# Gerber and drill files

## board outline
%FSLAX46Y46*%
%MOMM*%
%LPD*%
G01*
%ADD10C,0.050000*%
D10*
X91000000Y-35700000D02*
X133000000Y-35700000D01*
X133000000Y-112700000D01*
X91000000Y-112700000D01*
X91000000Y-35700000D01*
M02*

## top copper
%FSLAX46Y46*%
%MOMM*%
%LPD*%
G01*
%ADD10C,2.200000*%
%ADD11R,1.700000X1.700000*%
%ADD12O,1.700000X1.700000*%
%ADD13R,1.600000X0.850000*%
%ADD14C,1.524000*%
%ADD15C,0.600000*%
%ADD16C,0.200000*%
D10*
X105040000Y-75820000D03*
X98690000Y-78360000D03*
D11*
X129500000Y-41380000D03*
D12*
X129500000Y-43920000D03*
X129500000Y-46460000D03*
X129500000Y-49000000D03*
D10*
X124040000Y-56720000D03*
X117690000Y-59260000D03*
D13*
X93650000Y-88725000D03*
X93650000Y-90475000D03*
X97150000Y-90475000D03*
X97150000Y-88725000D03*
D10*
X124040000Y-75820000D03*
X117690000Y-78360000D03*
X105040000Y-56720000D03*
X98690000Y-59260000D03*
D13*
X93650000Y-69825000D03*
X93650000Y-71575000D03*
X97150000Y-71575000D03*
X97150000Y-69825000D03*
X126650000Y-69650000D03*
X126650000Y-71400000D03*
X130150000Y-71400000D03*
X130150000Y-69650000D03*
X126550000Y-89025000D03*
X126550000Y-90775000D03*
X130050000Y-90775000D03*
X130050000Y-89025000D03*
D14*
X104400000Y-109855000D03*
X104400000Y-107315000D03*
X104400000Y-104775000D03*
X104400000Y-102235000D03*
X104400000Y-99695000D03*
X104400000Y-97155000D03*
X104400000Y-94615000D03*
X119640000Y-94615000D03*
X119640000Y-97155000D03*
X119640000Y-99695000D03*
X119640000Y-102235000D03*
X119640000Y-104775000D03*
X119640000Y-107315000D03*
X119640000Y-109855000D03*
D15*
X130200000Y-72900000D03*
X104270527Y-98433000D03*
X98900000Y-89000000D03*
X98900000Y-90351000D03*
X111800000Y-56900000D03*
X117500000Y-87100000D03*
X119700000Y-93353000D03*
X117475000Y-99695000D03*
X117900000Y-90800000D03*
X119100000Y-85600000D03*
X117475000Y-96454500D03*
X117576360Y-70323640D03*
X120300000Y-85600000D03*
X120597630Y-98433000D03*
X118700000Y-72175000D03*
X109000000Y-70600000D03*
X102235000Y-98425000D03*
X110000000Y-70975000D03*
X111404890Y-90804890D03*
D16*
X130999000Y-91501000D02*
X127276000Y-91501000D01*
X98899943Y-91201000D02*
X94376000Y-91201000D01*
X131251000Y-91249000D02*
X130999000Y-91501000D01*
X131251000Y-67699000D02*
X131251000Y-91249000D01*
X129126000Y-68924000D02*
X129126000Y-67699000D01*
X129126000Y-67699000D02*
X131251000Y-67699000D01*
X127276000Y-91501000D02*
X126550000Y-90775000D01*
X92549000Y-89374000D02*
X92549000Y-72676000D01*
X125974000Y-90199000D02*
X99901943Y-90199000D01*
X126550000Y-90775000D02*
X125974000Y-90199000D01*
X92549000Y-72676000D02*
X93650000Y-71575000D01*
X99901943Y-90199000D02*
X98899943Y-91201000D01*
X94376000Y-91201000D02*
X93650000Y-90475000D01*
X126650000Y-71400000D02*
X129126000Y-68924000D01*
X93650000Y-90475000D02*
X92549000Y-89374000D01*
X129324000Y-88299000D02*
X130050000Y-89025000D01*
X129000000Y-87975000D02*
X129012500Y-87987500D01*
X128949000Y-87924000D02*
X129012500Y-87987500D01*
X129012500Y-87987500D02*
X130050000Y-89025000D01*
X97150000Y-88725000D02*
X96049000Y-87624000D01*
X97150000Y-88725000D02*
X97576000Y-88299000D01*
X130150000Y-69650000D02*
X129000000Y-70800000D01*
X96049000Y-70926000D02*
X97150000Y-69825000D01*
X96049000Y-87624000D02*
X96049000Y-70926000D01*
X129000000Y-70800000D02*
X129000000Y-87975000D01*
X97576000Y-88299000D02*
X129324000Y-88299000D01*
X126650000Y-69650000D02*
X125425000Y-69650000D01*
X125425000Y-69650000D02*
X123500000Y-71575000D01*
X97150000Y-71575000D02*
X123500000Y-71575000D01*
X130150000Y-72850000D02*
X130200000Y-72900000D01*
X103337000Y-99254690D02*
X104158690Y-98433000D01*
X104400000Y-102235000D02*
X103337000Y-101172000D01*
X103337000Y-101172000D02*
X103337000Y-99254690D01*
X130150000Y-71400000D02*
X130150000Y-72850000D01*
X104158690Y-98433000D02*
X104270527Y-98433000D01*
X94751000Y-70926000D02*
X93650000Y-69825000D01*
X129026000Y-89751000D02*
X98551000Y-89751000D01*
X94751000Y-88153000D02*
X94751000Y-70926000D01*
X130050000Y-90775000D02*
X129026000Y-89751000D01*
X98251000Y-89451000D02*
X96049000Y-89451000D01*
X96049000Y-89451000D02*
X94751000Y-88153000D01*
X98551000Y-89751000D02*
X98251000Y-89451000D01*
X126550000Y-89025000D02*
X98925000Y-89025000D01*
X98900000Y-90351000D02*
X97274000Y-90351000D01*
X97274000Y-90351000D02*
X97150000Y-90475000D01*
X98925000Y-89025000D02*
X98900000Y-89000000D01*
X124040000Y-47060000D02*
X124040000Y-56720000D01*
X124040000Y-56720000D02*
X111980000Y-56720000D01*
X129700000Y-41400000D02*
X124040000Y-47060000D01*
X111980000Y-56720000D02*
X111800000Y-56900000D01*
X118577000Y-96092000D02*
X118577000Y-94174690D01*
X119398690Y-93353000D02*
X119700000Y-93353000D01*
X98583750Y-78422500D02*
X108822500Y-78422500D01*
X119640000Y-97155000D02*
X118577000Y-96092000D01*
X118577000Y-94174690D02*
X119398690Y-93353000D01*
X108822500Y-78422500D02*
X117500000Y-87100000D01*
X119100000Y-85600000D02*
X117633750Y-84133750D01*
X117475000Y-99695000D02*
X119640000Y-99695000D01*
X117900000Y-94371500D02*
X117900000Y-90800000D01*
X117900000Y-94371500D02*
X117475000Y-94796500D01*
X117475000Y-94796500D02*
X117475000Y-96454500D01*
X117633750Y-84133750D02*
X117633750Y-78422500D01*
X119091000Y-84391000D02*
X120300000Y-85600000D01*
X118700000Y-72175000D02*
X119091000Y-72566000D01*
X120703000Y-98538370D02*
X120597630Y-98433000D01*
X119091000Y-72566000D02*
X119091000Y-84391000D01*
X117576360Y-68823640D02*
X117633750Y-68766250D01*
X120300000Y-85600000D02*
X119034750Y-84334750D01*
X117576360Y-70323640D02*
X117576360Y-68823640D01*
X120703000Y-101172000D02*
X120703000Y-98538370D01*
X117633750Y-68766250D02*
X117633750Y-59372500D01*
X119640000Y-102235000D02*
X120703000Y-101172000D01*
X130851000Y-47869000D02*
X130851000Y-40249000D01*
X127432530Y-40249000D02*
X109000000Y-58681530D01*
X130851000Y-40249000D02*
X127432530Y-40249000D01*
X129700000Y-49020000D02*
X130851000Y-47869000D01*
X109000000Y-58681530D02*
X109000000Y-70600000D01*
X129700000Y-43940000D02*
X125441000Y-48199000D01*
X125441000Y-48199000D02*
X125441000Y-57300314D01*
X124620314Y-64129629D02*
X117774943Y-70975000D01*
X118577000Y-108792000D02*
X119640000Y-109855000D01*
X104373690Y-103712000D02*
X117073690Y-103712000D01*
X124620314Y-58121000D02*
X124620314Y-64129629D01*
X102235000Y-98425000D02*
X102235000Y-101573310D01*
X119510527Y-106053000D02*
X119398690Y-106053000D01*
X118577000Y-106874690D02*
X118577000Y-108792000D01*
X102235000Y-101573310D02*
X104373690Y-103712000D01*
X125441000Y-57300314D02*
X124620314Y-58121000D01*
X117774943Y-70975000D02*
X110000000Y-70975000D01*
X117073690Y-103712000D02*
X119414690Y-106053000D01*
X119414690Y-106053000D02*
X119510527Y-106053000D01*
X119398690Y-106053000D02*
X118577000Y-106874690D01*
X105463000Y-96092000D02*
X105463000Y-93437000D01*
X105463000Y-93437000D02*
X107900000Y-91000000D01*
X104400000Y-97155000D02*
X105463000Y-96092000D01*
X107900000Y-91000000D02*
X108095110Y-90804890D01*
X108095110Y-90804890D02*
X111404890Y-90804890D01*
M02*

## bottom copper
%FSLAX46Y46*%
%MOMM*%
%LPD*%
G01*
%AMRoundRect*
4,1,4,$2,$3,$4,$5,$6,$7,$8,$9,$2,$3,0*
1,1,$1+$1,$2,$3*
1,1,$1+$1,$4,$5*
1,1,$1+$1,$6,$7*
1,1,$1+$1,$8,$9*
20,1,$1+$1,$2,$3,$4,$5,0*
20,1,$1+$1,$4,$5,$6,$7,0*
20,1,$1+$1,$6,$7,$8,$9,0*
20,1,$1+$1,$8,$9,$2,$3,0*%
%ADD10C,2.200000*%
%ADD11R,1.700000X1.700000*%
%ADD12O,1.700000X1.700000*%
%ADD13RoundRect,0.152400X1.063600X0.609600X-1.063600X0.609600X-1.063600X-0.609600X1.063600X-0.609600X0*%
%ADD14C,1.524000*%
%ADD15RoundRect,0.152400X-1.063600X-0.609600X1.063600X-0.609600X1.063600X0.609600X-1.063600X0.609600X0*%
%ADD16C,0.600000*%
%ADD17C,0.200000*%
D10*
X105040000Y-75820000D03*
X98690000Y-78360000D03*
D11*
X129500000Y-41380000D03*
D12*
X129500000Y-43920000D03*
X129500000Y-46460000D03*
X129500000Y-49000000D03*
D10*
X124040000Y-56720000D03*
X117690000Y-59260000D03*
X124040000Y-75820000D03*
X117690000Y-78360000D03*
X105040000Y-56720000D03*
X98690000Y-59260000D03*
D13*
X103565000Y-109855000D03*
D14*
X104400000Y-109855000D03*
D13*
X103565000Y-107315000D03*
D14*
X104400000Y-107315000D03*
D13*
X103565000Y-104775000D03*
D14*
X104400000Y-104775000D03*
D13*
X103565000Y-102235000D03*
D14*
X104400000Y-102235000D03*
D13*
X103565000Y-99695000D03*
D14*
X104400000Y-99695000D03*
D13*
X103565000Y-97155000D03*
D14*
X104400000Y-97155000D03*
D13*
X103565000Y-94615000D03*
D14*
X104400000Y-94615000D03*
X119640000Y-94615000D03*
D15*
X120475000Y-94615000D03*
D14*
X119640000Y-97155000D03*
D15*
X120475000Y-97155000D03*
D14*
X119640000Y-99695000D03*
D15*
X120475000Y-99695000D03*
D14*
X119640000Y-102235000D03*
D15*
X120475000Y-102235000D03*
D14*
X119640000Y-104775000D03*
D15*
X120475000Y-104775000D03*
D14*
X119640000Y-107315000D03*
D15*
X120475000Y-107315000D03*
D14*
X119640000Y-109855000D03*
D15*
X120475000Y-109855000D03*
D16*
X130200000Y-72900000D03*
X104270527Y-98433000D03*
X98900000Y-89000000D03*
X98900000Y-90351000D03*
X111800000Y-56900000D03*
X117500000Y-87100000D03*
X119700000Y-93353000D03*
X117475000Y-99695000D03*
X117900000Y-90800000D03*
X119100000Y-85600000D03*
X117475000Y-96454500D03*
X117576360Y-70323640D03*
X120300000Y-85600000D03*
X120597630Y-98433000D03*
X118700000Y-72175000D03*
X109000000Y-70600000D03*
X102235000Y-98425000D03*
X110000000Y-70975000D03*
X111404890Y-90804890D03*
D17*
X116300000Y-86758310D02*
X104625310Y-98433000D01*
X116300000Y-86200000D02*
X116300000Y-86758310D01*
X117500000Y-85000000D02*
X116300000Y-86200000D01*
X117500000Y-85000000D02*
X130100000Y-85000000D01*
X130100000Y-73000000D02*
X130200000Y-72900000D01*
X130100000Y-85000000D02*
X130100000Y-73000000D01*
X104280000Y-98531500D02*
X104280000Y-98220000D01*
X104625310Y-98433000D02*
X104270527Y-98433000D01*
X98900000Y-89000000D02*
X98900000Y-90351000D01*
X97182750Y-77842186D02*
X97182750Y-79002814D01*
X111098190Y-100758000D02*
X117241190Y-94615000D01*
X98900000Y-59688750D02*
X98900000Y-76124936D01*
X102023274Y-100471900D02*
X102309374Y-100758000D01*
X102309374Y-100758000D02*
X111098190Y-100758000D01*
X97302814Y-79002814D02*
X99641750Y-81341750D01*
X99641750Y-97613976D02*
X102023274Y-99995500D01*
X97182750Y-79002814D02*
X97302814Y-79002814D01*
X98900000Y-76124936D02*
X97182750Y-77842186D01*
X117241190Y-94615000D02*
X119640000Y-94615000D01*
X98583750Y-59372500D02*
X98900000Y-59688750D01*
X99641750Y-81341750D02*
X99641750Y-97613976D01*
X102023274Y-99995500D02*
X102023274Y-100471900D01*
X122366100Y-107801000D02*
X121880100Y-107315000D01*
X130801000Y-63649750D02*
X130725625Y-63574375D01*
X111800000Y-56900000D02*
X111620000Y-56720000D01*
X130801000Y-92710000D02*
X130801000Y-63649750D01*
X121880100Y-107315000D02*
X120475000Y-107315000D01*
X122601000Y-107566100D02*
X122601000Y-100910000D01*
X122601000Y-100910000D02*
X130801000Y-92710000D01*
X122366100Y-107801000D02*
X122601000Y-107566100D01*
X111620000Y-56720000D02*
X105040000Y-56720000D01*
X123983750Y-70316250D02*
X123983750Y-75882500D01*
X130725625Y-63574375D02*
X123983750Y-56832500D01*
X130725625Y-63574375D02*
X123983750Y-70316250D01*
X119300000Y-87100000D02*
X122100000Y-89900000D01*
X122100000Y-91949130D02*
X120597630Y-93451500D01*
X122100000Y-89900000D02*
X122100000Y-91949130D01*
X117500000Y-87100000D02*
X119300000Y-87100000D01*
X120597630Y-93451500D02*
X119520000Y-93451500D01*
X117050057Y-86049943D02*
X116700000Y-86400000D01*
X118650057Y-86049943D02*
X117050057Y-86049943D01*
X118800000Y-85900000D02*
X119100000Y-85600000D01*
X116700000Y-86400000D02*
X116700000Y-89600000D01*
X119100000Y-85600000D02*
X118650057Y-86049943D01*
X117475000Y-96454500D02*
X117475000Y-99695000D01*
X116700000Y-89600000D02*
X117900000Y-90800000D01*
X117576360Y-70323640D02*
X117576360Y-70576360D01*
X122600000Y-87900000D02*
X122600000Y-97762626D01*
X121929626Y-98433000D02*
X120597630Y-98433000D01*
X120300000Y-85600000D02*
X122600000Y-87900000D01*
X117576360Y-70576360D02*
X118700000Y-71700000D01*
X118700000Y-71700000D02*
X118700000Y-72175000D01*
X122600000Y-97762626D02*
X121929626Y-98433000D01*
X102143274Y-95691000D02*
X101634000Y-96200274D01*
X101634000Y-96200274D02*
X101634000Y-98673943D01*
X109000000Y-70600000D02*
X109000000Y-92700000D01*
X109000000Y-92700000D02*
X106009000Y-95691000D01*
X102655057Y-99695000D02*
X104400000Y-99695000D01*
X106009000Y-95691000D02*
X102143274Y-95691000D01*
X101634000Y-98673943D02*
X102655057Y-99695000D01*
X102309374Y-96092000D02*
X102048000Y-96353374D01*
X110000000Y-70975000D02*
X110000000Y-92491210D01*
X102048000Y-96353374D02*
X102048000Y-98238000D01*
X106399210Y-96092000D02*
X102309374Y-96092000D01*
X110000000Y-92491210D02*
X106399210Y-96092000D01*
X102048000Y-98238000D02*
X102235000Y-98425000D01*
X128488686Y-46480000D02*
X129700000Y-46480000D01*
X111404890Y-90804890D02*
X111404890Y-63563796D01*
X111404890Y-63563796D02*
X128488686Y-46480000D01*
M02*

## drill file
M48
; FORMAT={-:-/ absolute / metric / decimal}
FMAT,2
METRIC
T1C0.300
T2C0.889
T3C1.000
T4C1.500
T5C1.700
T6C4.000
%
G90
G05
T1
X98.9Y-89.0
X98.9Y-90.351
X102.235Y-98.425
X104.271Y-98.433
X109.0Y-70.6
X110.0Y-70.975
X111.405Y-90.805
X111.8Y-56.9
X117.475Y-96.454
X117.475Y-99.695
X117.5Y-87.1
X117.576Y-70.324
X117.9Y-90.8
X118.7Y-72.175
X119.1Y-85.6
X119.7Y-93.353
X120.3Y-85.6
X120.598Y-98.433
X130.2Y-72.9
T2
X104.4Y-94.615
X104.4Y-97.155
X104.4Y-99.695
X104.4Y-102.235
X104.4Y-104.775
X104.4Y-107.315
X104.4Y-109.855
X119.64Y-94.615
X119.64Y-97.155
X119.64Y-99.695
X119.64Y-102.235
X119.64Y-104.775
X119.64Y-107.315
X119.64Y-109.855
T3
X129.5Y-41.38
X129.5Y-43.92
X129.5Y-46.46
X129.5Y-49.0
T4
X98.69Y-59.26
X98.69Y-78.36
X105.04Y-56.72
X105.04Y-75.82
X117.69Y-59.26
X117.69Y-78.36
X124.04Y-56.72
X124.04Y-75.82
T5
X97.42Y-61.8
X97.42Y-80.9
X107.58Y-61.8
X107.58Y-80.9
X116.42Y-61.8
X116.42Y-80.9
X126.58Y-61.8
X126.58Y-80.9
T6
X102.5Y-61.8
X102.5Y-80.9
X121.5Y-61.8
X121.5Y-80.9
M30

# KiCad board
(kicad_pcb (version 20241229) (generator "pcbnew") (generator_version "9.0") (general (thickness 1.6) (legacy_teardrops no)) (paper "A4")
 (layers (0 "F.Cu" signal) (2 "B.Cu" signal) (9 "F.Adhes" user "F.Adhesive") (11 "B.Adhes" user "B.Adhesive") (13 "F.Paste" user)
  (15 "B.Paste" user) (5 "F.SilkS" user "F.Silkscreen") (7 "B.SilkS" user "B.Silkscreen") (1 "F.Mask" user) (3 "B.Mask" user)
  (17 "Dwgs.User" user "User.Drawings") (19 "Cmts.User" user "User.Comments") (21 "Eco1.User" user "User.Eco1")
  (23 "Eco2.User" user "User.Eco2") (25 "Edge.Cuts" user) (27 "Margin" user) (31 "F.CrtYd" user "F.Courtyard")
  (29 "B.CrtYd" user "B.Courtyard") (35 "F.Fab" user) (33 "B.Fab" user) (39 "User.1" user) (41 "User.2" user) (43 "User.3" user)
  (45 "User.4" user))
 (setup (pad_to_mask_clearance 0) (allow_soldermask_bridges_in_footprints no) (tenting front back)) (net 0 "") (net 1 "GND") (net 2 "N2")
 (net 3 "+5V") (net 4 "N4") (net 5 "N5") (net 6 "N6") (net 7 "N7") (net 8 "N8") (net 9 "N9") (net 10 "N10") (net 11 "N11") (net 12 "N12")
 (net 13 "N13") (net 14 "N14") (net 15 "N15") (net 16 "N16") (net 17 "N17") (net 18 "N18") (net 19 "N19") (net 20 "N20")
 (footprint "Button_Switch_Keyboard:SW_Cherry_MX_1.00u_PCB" (layer "F.Cu") (at 105.04 75.82)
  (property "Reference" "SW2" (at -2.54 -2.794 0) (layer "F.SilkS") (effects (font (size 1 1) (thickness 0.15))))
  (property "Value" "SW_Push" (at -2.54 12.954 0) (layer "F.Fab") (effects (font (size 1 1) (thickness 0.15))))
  (pad "" np_thru_hole circle (at -7.62 5.08) (size 1.7 1.7) (drill 1.7) (layers "*.Cu" "*.Mask"))
  (pad "" np_thru_hole circle (at -2.54 5.08) (size 4 4) (drill 4) (layers "*.Cu" "*.Mask"))
  (pad "" np_thru_hole circle (at 2.54 5.08) (size 1.7 1.7) (drill 1.7) (layers "*.Cu" "*.Mask"))
  (pad "1" thru_hole circle (at 0 0) (size 2.2 2.2) (drill 1.5) (layers "*.Cu" "*.Mask") (remove_unused_layers no) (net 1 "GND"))
  (pad "2" thru_hole circle (at -6.35 2.54) (size 2.2 2.2) (drill 1.5) (layers "*.Cu" "*.Mask") (remove_unused_layers no) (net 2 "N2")))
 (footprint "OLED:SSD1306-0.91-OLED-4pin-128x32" (layer "F.Cu") (at 93 39.19)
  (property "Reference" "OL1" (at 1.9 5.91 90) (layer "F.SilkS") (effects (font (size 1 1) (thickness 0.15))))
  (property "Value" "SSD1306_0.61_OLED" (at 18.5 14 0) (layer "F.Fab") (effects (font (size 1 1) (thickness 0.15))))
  (pad "1" thru_hole rect (at 36.5 2.19) (size 1.7 1.7) (drill 1) (layers "*.Cu" "*.Mask") (remove_unused_layers no) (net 1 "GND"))
  (pad "2" thru_hole oval (at 36.5 4.73) (size 1.7 1.7) (drill 1) (layers "*.Cu" "*.Mask") (remove_unused_layers no) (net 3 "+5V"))
  (pad "3" thru_hole oval (at 36.5 7.27) (size 1.7 1.7) (drill 1) (layers "*.Cu" "*.Mask") (remove_unused_layers no) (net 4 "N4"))
  (pad "4" thru_hole oval (at 36.5 9.81) (size 1.7 1.7) (drill 1) (layers "*.Cu" "*.Mask") (remove_unused_layers no) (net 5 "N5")))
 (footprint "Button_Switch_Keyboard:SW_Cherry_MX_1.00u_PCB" (layer "F.Cu") (at 124.04 56.72)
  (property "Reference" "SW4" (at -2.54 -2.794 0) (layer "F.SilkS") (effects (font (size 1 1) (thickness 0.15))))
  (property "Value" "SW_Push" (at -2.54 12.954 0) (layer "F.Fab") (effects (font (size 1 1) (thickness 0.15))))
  (pad "" np_thru_hole circle (at -7.62 5.08) (size 1.7 1.7) (drill 1.7) (layers "*.Cu" "*.Mask"))
  (pad "" np_thru_hole circle (at -2.54 5.08) (size 4 4) (drill 4) (layers "*.Cu" "*.Mask"))
  (pad "" np_thru_hole circle (at 2.54 5.08) (size 1.7 1.7) (drill 1.7) (layers "*.Cu" "*.Mask"))
  (pad "1" thru_hole circle (at 0 0) (size 2.2 2.2) (drill 1.5) (layers "*.Cu" "*.Mask") (remove_unused_layers no) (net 1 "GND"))
  (pad "2" thru_hole circle (at -6.35 2.54) (size 2.2 2.2) (drill 1.5) (layers "*.Cu" "*.Mask") (remove_unused_layers no) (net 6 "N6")))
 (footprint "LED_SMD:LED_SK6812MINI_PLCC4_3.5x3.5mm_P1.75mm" (layer "F.Cu") (at 95.4 89.6)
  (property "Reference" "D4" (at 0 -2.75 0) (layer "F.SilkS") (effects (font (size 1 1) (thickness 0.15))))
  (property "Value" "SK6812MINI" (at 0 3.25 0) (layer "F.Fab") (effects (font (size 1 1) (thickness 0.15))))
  (pad "1" smd rect (at -1.75 -0.875) (size 1.6 0.85) (layers "F.Cu" "F.Mask" "F.Paste") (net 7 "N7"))
  (pad "2" smd rect (at -1.75 0.875) (size 1.6 0.85) (layers "F.Cu" "F.Mask" "F.Paste") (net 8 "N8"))
  (pad "3" smd rect (at 1.75 0.875) (size 1.6 0.85) (layers "F.Cu" "F.Mask" "F.Paste") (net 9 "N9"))
  (pad "4" smd rect (at 1.75 -0.875) (size 1.6 0.85) (layers "F.Cu" "F.Mask" "F.Paste") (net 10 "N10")))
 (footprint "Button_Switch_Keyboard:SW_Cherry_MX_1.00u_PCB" (layer "F.Cu") (at 124.04 75.82)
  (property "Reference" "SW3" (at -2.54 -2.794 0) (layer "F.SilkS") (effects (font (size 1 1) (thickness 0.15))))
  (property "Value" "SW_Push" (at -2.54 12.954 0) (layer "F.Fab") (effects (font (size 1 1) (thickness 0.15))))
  (pad "" np_thru_hole circle (at -7.62 5.08) (size 1.7 1.7) (drill 1.7) (layers "*.Cu" "*.Mask"))
  (pad "" np_thru_hole circle (at -2.54 5.08) (size 4 4) (drill 4) (layers "*.Cu" "*.Mask"))
  (pad "" np_thru_hole circle (at 2.54 5.08) (size 1.7 1.7) (drill 1.7) (layers "*.Cu" "*.Mask"))
  (pad "1" thru_hole circle (at 0 0) (size 2.2 2.2) (drill 1.5) (layers "*.Cu" "*.Mask") (remove_unused_layers no) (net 1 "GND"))
  (pad "2" thru_hole circle (at -6.35 2.54) (size 2.2 2.2) (drill 1.5) (layers "*.Cu" "*.Mask") (remove_unused_layers no) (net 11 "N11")))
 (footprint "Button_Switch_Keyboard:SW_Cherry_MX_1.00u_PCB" (layer "F.Cu") (at 105.04 56.72)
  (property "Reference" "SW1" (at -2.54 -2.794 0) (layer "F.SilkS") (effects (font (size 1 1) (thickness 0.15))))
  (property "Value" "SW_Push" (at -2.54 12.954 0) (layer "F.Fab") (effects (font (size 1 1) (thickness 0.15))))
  (pad "" np_thru_hole circle (at -7.62 5.08) (size 1.7 1.7) (drill 1.7) (layers "*.Cu" "*.Mask"))
  (pad "" np_thru_hole circle (at -2.54 5.08) (size 4 4) (drill 4) (layers "*.Cu" "*.Mask"))
  (pad "" np_thru_hole circle (at 2.54 5.08) (size 1.7 1.7) (drill 1.7) (layers "*.Cu" "*.Mask"))
  (pad "1" thru_hole circle (at 0 0) (size 2.2 2.2) (drill 1.5) (layers "*.Cu" "*.Mask") (remove_unused_layers no) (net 1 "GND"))
  (pad "2" thru_hole circle (at -6.35 2.54) (size 2.2 2.2) (drill 1.5) (layers "*.Cu" "*.Mask") (remove_unused_layers no) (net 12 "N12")))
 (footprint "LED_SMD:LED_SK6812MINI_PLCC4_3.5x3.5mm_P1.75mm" (layer "F.Cu") (at 95.4 70.7)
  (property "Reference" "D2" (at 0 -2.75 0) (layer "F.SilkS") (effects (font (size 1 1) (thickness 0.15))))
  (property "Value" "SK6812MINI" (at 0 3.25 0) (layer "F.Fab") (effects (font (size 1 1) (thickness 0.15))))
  (pad "1" smd rect (at -1.75 -0.875) (size 1.6 0.85) (layers "F.Cu" "F.Mask" "F.Paste") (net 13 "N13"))
  (pad "2" smd rect (at -1.75 0.875) (size 1.6 0.85) (layers "F.Cu" "F.Mask" "F.Paste") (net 8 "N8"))
  (pad "3" smd rect (at 1.75 0.875) (size 1.6 0.85) (layers "F.Cu" "F.Mask" "F.Paste") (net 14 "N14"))
  (pad "4" smd rect (at 1.75 -0.875) (size 1.6 0.85) (layers "F.Cu" "F.Mask" "F.Paste") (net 10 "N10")))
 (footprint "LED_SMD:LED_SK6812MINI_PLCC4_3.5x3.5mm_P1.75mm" (layer "F.Cu") (at 128.4 70.525)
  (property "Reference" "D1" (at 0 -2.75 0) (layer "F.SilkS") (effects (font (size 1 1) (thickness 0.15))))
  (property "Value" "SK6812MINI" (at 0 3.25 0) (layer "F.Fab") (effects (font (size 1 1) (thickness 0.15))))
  (pad "1" smd rect (at -1.75 -0.875) (size 1.6 0.85) (layers "F.Cu" "F.Mask" "F.Paste") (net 14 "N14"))
  (pad "2" smd rect (at -1.75 0.875) (size 1.6 0.85) (layers "F.Cu" "F.Mask" "F.Paste") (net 8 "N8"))
  (pad "3" smd rect (at 1.75 0.875) (size 1.6 0.85) (layers "F.Cu" "F.Mask" "F.Paste") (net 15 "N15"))
  (pad "4" smd rect (at 1.75 -0.875) (size 1.6 0.85) (layers "F.Cu" "F.Mask" "F.Paste") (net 10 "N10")))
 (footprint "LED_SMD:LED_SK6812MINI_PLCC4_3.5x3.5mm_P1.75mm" (layer "F.Cu") (at 128.3 89.9)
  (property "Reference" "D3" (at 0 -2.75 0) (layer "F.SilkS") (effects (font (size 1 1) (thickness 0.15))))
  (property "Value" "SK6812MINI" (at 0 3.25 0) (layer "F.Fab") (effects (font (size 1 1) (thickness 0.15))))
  (pad "1" smd rect (at -1.75 -0.875) (size 1.6 0.85) (layers "F.Cu" "F.Mask" "F.Paste") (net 9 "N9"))
  (pad "2" smd rect (at -1.75 0.875) (size 1.6 0.85) (layers "F.Cu" "F.Mask" "F.Paste") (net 8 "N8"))
  (pad "3" smd rect (at 1.75 0.875) (size 1.6 0.85) (layers "F.Cu" "F.Mask" "F.Paste") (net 13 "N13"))
  (pad "4" smd rect (at 1.75 -0.875) (size 1.6 0.85) (layers "F.Cu" "F.Mask" "F.Paste") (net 10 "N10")))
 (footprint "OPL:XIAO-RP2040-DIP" (layer "B.Cu") (at 112.02 102.235)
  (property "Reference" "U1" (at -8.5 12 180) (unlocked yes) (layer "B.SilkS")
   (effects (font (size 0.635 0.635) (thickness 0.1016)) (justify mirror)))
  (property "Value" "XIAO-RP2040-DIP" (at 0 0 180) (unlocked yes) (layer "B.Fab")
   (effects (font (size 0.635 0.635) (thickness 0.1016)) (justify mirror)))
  (pad "1" smd roundrect (at -8.455 7.62 180) (size 2.432 1.524) (layers "B.Cu" "B.Mask") (roundrect_rratio 0.1) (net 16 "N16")
   (thermal_bridge_angle 45))
  (pad "1" thru_hole circle (at -7.62 7.62 180) (size 1.524 1.524) (drill 0.889) (layers "*.Cu" "*.Mask") (remove_unused_layers no)
   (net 16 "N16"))
  (pad "2" smd roundrect (at -8.455 5.08 180) (size 2.432 1.524) (layers "B.Cu" "B.Mask") (roundrect_rratio 0.1) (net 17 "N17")
   (thermal_bridge_angle 45))
  (pad "2" thru_hole circle (at -7.62 5.08 180) (size 1.524 1.524) (drill 0.889) (layers "*.Cu" "*.Mask") (remove_unused_layers no)
   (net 17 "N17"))
  (pad "3" smd roundrect (at -8.455 2.54 180) (size 2.432 1.524) (layers "B.Cu" "B.Mask") (roundrect_rratio 0.1) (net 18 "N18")
   (thermal_bridge_angle 45))
  (pad "3" thru_hole circle (at -7.62 2.54 180) (size 1.524 1.524) (drill 0.889) (layers "*.Cu" "*.Mask") (remove_unused_layers no)
   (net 18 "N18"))
  (pad "4" smd roundrect (at -8.455 0 180) (size 2.432 1.524) (layers "B.Cu" "B.Mask") (roundrect_rratio 0.1) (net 15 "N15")
   (thermal_bridge_angle 45))
  (pad "4" thru_hole circle (at -7.62 0 180) (size 1.524 1.524) (drill 0.889) (layers "*.Cu" "*.Mask") (remove_unused_layers no)
   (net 15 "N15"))
  (pad "5" smd roundrect (at -8.455 -2.54 180) (size 2.432 1.524) (layers "B.Cu" "B.Mask") (roundrect_rratio 0.1) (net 5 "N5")
   (thermal_bridge_angle 45))
  (pad "5" thru_hole circle (at -7.62 -2.54 180) (size 1.524 1.524) (drill 0.889) (layers "*.Cu" "*.Mask") (remove_unused_layers no)
   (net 5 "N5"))
  (pad "6" smd roundrect (at -8.455 -5.08 180) (size 2.432 1.524) (layers "B.Cu" "B.Mask") (roundrect_rratio 0.1) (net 4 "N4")
   (thermal_bridge_angle 45))
  (pad "6" thru_hole circle (at -7.62 -5.08 180) (size 1.524 1.524) (drill 0.889) (layers "*.Cu" "*.Mask") (remove_unused_layers no)
   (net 4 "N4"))
  (pad "7" smd roundrect (at -8.455 -7.62 180) (size 2.432 1.524) (layers "B.Cu" "B.Mask") (roundrect_rratio 0.1) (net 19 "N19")
   (thermal_bridge_angle 45))
  (pad "7" thru_hole circle (at -7.62 -7.62 180) (size 1.524 1.524) (drill 0.889) (layers "*.Cu" "*.Mask") (remove_unused_layers no)
   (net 19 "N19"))
  (pad "8" thru_hole circle (at 7.62 -7.62) (size 1.524 1.524) (drill 0.889) (layers "*.Cu" "*.Mask") (remove_unused_layers no)
   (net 12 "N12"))
  (pad "8" smd roundrect (at 8.455 -7.62) (size 2.432 1.524) (layers "B.Cu" "B.Mask") (roundrect_rratio 0.1) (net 12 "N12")
   (thermal_bridge_angle 45))
  (pad "9" thru_hole circle (at 7.62 -5.08) (size 1.524 1.524) (drill 0.889) (layers "*.Cu" "*.Mask") (remove_unused_layers no) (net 2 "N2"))
  (pad "9" smd roundrect (at 8.455 -5.08) (size 2.432 1.524) (layers "B.Cu" "B.Mask") (roundrect_rratio 0.1) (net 2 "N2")
   (thermal_bridge_angle 45))
  (pad "10" thru_hole circle (at 7.62 -2.54) (size 1.524 1.524) (drill 0.889) (layers "*.Cu" "*.Mask") (remove_unused_layers no)
   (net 11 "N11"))
  (pad "10" smd roundrect (at 8.455 -2.54) (size 2.432 1.524) (layers "B.Cu" "B.Mask") (roundrect_rratio 0.1) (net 11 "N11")
   (thermal_bridge_angle 45))
  (pad "11" thru_hole circle (at 7.62 0) (size 1.524 1.524) (drill 0.889) (layers "*.Cu" "*.Mask") (remove_unused_layers no) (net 6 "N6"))
  (pad "11" smd roundrect (at 8.455 0) (size 2.432 1.524) (layers "B.Cu" "B.Mask") (roundrect_rratio 0.1) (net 6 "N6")
   (thermal_bridge_angle 45))
  (pad "12" thru_hole circle (at 7.62 2.54) (size 1.524 1.524) (drill 0.889) (layers "*.Cu" "*.Mask") (remove_unused_layers no)
   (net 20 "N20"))
  (pad "12" smd roundrect (at 8.455 2.54) (size 2.432 1.524) (layers "B.Cu" "B.Mask") (roundrect_rratio 0.1) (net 20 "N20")
   (thermal_bridge_angle 45))
  (pad "13" thru_hole circle (at 7.62 5.08) (size 1.524 1.524) (drill 0.889) (layers "*.Cu" "*.Mask") (remove_unused_layers no)
   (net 1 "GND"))
  (pad "13" smd roundrect (at 8.455 5.08) (size 2.432 1.524) (layers "B.Cu" "B.Mask") (roundrect_rratio 0.1) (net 1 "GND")
   (thermal_bridge_angle 45))
  (pad "14" thru_hole circle (at 7.62 7.62) (size 1.524 1.524) (drill 0.889) (layers "*.Cu" "*.Mask") (remove_unused_layers no)
   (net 3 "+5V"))
  (pad "14" smd roundrect (at 8.455 7.62) (size 2.432 1.524) (layers "B.Cu" "B.Mask") (roundrect_rratio 0.1) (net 3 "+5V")
   (thermal_bridge_angle 45)))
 (gr_rect (start 91 35.7) (end 133 112.7) (stroke (width 0.05) (type default)) (fill no) (layer "Edge.Cuts"))
 (segment (start 130.999 91.501) (end 127.276 91.501) (width 0.2) (layer "F.Cu") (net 8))
 (segment (start 98.899943 91.201) (end 94.376 91.201) (width 0.2) (layer "F.Cu") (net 8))
 (segment (start 131.251 91.249) (end 130.999 91.501) (width 0.2) (layer "F.Cu") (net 8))
 (segment (start 131.251 67.699) (end 131.251 91.249) (width 0.2) (layer "F.Cu") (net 8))
 (segment (start 129.126 68.924) (end 129.126 67.699) (width 0.2) (layer "F.Cu") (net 8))
 (segment (start 129.126 67.699) (end 131.251 67.699) (width 0.2) (layer "F.Cu") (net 8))
 (segment (start 127.276 91.501) (end 126.55 90.775) (width 0.2) (layer "F.Cu") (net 8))
 (segment (start 92.549 89.374) (end 92.549 72.676) (width 0.2) (layer "F.Cu") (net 8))
 (segment (start 125.974 90.199) (end 99.901943 90.199) (width 0.2) (layer "F.Cu") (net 8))
 (segment (start 126.55 90.775) (end 125.974 90.199) (width 0.2) (layer "F.Cu") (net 8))
 (segment (start 92.549 72.676) (end 93.65 71.575) (width 0.2) (layer "F.Cu") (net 8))
 (segment (start 99.901943 90.199) (end 98.899943 91.201) (width 0.2) (layer "F.Cu") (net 8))
 (segment (start 94.376 91.201) (end 93.65 90.475) (width 0.2) (layer "F.Cu") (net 8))
 (segment (start 126.65 71.4) (end 129.126 68.924) (width 0.2) (layer "F.Cu") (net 8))
 (segment (start 93.65 90.475) (end 92.549 89.374) (width 0.2) (layer "F.Cu") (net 8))
 (segment (start 129.324 88.299) (end 130.05 89.025) (width 0.2) (layer "F.Cu") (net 10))
 (segment (start 129 87.975) (end 129.0125 87.9875) (width 0.2) (layer "F.Cu") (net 10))
 (segment (start 128.949 87.924) (end 129.0125 87.9875) (width 0.2) (layer "F.Cu") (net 10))
 (segment (start 129.0125 87.9875) (end 130.05 89.025) (width 0.2) (layer "F.Cu") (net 10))
 (segment (start 97.15 88.725) (end 96.049 87.624) (width 0.2) (layer "F.Cu") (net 10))
 (segment (start 97.15 88.725) (end 97.576 88.299) (width 0.2) (layer "F.Cu") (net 10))
 (segment (start 130.15 69.65) (end 129 70.8) (width 0.2) (layer "F.Cu") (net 10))
 (segment (start 96.049 70.926) (end 97.15 69.825) (width 0.2) (layer "F.Cu") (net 10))
 (segment (start 96.049 87.624) (end 96.049 70.926) (width 0.2) (layer "F.Cu") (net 10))
 (segment (start 129 70.8) (end 129 87.975) (width 0.2) (layer "F.Cu") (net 10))
 (segment (start 97.576 88.299) (end 129.324 88.299) (width 0.2) (layer "F.Cu") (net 10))
 (segment (start 126.65 69.65) (end 125.425 69.65) (width 0.2) (layer "F.Cu") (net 14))
 (segment (start 125.425 69.65) (end 123.5 71.575) (width 0.2) (layer "F.Cu") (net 14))
 (segment (start 97.15 71.575) (end 123.5 71.575) (width 0.2) (layer "F.Cu") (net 14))
 (segment (start 130.15 72.85) (end 130.2 72.9) (width 0.2) (layer "F.Cu") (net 15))
 (segment (start 103.337 99.25469) (end 104.15869 98.433) (width 0.2) (layer "F.Cu") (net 15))
 (segment (start 104.4 102.235) (end 103.337 101.172) (width 0.2) (layer "F.Cu") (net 15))
 (segment (start 103.337 101.172) (end 103.337 99.25469) (width 0.2) (layer "F.Cu") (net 15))
 (segment (start 130.15 71.4) (end 130.15 72.85) (width 0.2) (layer "F.Cu") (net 15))
 (segment (start 104.15869 98.433) (end 104.270527 98.433) (width 0.2) (layer "F.Cu") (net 15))
 (via (at 130.2 72.9) (size 0.6) (drill 0.3) (layers "F.Cu" "B.Cu") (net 15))
 (via (at 104.270527 98.433) (size 0.6) (drill 0.3) (layers "F.Cu" "B.Cu") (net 15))
 (segment (start 116.3 86.75831) (end 104.62531 98.433) (width 0.2) (layer "B.Cu") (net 15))
 (segment (start 116.3 86.2) (end 116.3 86.75831) (width 0.2) (layer "B.Cu") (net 15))
 (segment (start 117.5 85) (end 116.3 86.2) (width 0.2) (layer "B.Cu") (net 15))
 (segment (start 117.5 85) (end 130.1 85) (width 0.2) (layer "B.Cu") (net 15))
 (segment (start 130.1 73) (end 130.2 72.9) (width 0.2) (layer "B.Cu") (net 15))
 (segment (start 130.1 85) (end 130.1 73) (width 0.2) (layer "B.Cu") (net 15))
 (segment (start 104.28 98.5315) (end 104.28 98.22) (width 0.2) (layer "B.Cu") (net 15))
 (segment (start 104.62531 98.433) (end 104.270527 98.433) (width 0.2) (layer "B.Cu") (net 15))
 (segment (start 94.751 70.926) (end 93.65 69.825) (width 0.2) (layer "F.Cu") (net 13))
 (segment (start 129.026 89.751) (end 98.551 89.751) (width 0.2) (layer "F.Cu") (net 13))
 (segment (start 94.751 88.153) (end 94.751 70.926) (width 0.2) (layer "F.Cu") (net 13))
 (segment (start 130.05 90.775) (end 129.026 89.751) (width 0.2) (layer "F.Cu") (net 13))
 (segment (start 98.251 89.451) (end 96.049 89.451) (width 0.2) (layer "F.Cu") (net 13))
 (segment (start 96.049 89.451) (end 94.751 88.153) (width 0.2) (layer "F.Cu") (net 13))
 (segment (start 98.551 89.751) (end 98.251 89.451) (width 0.2) (layer "F.Cu") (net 13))
 (segment (start 126.55 89.025) (end 98.925 89.025) (width 0.2) (layer "F.Cu") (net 9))
 (segment (start 98.9 90.351) (end 97.274 90.351) (width 0.2) (layer "F.Cu") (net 9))
 (segment (start 97.274 90.351) (end 97.15 90.475) (width 0.2) (layer "F.Cu") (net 9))
 (segment (start 98.925 89.025) (end 98.9 89) (width 0.2) (layer "F.Cu") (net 9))
 (via (at 98.9 89) (size 0.6) (drill 0.3) (layers "F.Cu" "B.Cu") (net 9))
 (via (at 98.9 90.351) (size 0.6) (drill 0.3) (layers "F.Cu" "B.Cu") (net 9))
 (segment (start 98.9 89) (end 98.9 90.351) (width 0.2) (layer "B.Cu") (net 9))
 (segment (start 97.18275 77.842186) (end 97.18275 79.002814) (width 0.2) (layer "B.Cu") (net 12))
 (segment (start 111.09819 100.758) (end 117.24119 94.615) (width 0.2) (layer "B.Cu") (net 12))
 (segment (start 98.9 59.68875) (end 98.9 76.124936) (width 0.2) (layer "B.Cu") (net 12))
 (segment (start 102.023274 100.4719) (end 102.309374 100.758) (width 0.2) (layer "B.Cu") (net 12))
 (segment (start 102.309374 100.758) (end 111.09819 100.758) (width 0.2) (layer "B.Cu") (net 12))
 (segment (start 97.302814 79.002814) (end 99.64175 81.34175) (width 0.2) (layer "B.Cu") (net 12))
 (segment (start 99.64175 97.613976) (end 102.023274 99.9955) (width 0.2) (layer "B.Cu") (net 12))
 (segment (start 97.18275 79.002814) (end 97.302814 79.002814) (width 0.2) (layer "B.Cu") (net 12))
 (segment (start 98.9 76.124936) (end 97.18275 77.842186) (width 0.2) (layer "B.Cu") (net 12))
 (segment (start 117.24119 94.615) (end 119.64 94.615) (width 0.2) (layer "B.Cu") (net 12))
 (segment (start 98.58375 59.3725) (end 98.9 59.68875) (width 0.2) (layer "B.Cu") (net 12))
 (segment (start 99.64175 81.34175) (end 99.64175 97.613976) (width 0.2) (layer "B.Cu") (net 12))
 (segment (start 102.023274 99.9955) (end 102.023274 100.4719) (width 0.2) (layer "B.Cu") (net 12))
 (segment (start 124.04 47.06) (end 124.04 56.72) (width 0.2) (layer "F.Cu") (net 1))
 (segment (start 124.04 56.72) (end 111.98 56.72) (width 0.2) (layer "F.Cu") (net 1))
 (segment (start 129.7 41.4) (end 124.04 47.06) (width 0.2) (layer "F.Cu") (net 1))
 (segment (start 111.98 56.72) (end 111.8 56.9) (width 0.2) (layer "F.Cu") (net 1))
 (via (at 111.8 56.9) (size 0.6) (drill 0.3) (layers "F.Cu" "B.Cu") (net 1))
 (segment (start 122.3661 107.801) (end 121.8801 107.315) (width 0.2) (layer "B.Cu") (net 1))
 (segment (start 130.801 63.64975) (end 130.725625 63.574375) (width 0.2) (layer "B.Cu") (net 1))
 (segment (start 111.8 56.9) (end 111.62 56.72) (width 0.2) (layer "B.Cu") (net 1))
 (segment (start 130.801 92.71) (end 130.801 63.64975) (width 0.2) (layer "B.Cu") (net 1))
 (segment (start 121.8801 107.315) (end 120.475 107.315) (width 0.2) (layer "B.Cu") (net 1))
 (segment (start 122.601 107.5661) (end 122.601 100.91) (width 0.2) (layer "B.Cu") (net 1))
 (segment (start 122.601 100.91) (end 130.801 92.71) (width 0.2) (layer "B.Cu") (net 1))
 (segment (start 122.3661 107.801) (end 122.601 107.5661) (width 0.2) (layer "B.Cu") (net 1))
 (segment (start 111.62 56.72) (end 105.04 56.72) (width 0.2) (layer "B.Cu") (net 1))
 (segment (start 123.98375 70.31625) (end 123.98375 75.8825) (width 0.2) (layer "B.Cu") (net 1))
 (segment (start 130.725625 63.574375) (end 123.98375 56.8325) (width 0.2) (layer "B.Cu") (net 1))
 (segment (start 130.725625 63.574375) (end 123.98375 70.31625) (width 0.2) (layer "B.Cu") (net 1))
 (segment (start 118.577 96.092) (end 118.577 94.17469) (width 0.2) (layer "F.Cu") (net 2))
 (segment (start 119.39869 93.353) (end 119.7 93.353) (width 0.2) (layer "F.Cu") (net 2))
 (segment (start 98.58375 78.4225) (end 108.8225 78.4225) (width 0.2) (layer "F.Cu") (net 2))
 (segment (start 119.64 97.155) (end 118.577 96.092) (width 0.2) (layer "F.Cu") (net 2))
 (segment (start 118.577 94.17469) (end 119.39869 93.353) (width 0.2) (layer "F.Cu") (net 2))
 (segment (start 108.8225 78.4225) (end 117.5 87.1) (width 0.2) (layer "F.Cu") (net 2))
 (via (at 117.5 87.1) (size 0.6) (drill 0.3) (layers "F.Cu" "B.Cu") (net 2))
 (via (at 119.7 93.353) (size 0.6) (drill 0.3) (layers "F.Cu" "B.Cu") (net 2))
 (segment (start 119.3 87.1) (end 122.1 89.9) (width 0.2) (layer "B.Cu") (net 2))
 (segment (start 122.1 91.94913) (end 120.59763 93.4515) (width 0.2) (layer "B.Cu") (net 2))
 (segment (start 122.1 89.9) (end 122.1 91.94913) (width 0.2) (layer "B.Cu") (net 2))
 (segment (start 117.5 87.1) (end 119.3 87.1) (width 0.2) (layer "B.Cu") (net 2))
 (segment (start 120.59763 93.4515) (end 119.52 93.4515) (width 0.2) (layer "B.Cu") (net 2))
 (segment (start 119.1 85.6) (end 117.63375 84.13375) (width 0.2) (layer "F.Cu") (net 11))
 (segment (start 117.475 99.695) (end 119.64 99.695) (width 0.2) (layer "F.Cu") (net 11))
 (segment (start 117.9 94.3715) (end 117.9 90.8) (width 0.2) (layer "F.Cu") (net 11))
 (segment (start 117.9 94.3715) (end 117.475 94.7965) (width 0.2) (layer "F.Cu") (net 11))
 (segment (start 117.475 94.7965) (end 117.475 96.4545) (width 0.2) (layer "F.Cu") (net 11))
 (segment (start 117.63375 84.13375) (end 117.63375 78.4225) (width 0.2) (layer "F.Cu") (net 11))
 (via (at 117.475 99.695) (size 0.6) (drill 0.3) (layers "F.Cu" "B.Cu") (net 11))
 (via (at 117.9 90.8) (size 0.6) (drill 0.3) (layers "F.Cu" "B.Cu") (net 11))
 (via (at 119.1 85.6) (size 0.6) (drill 0.3) (layers "F.Cu" "B.Cu") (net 11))
 (via (at 117.475 96.4545) (size 0.6) (drill 0.3) (layers "F.Cu" "B.Cu") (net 11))
 (segment (start 117.050057 86.049943) (end 116.7 86.4) (width 0.2) (layer "B.Cu") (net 11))
 (segment (start 118.650057 86.049943) (end 117.050057 86.049943) (width 0.2) (layer "B.Cu") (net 11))
 (segment (start 118.8 85.9) (end 119.1 85.6) (width 0.2) (layer "B.Cu") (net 11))
 (segment (start 116.7 86.4) (end 116.7 89.6) (width 0.2) (layer "B.Cu") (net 11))
 (segment (start 119.1 85.6) (end 118.650057 86.049943) (width 0.2) (layer "B.Cu") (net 11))
 (segment (start 117.475 96.4545) (end 117.475 99.695) (width 0.2) (layer "B.Cu") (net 11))
 (segment (start 116.7 89.6) (end 117.9 90.8) (width 0.2) (layer "B.Cu") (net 11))
 (segment (start 119.091 84.391) (end 120.3 85.6) (width 0.2) (layer "F.Cu") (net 6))
 (segment (start 118.7 72.175) (end 119.091 72.566) (width 0.2) (layer "F.Cu") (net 6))
 (segment (start 120.703 98.53837) (end 120.59763 98.433) (width 0.2) (layer "F.Cu") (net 6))
 (segment (start 119.091 72.566) (end 119.091 84.391) (width 0.2) (layer "F.Cu") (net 6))
 (segment (start 117.57636 68.82364) (end 117.63375 68.76625) (width 0.2) (layer "F.Cu") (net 6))
 (segment (start 120.3 85.6) (end 119.03475 84.33475) (width 0.2) (layer "F.Cu") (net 6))
 (segment (start 117.57636 70.32364) (end 117.57636 68.82364) (width 0.2) (layer "F.Cu") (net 6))
 (segment (start 120.703 101.172) (end 120.703 98.53837) (width 0.2) (layer "F.Cu") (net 6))
 (segment (start 117.63375 68.76625) (end 117.63375 59.3725) (width 0.2) (layer "F.Cu") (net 6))
 (segment (start 119.64 102.235) (end 120.703 101.172) (width 0.2) (layer "F.Cu") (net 6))
 (via (at 117.57636 70.32364) (size 0.6) (drill 0.3) (layers "F.Cu" "B.Cu") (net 6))
 (via (at 120.3 85.6) (size 0.6) (drill 0.3) (layers "F.Cu" "B.Cu") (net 6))
 (via (at 120.59763 98.433) (size 0.6) (drill 0.3) (layers "F.Cu" "B.Cu") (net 6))
 (via (at 118.7 72.175) (size 0.6) (drill 0.3) (layers "F.Cu" "B.Cu") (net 6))
 (segment (start 117.57636 70.32364) (end 117.57636 70.57636) (width 0.2) (layer "B.Cu") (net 6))
 (segment (start 122.6 87.9) (end 122.6 97.762626) (width 0.2) (layer "B.Cu") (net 6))
 (segment (start 121.929626 98.433) (end 120.59763 98.433) (width 0.2) (layer "B.Cu") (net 6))
 (segment (start 120.3 85.6) (end 122.6 87.9) (width 0.2) (layer "B.Cu") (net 6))
 (segment (start 117.57636 70.57636) (end 118.7 71.7) (width 0.2) (layer "B.Cu") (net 6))
 (segment (start 118.7 71.7) (end 118.7 72.175) (width 0.2) (layer "B.Cu") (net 6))
 (segment (start 122.6 97.762626) (end 121.929626 98.433) (width 0.2) (layer "B.Cu") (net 6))
 (segment (start 130.851 47.869) (end 130.851 40.249) (width 0.2) (layer "F.Cu") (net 5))
 (segment (start 127.43253 40.249) (end 109 58.68153) (width 0.2) (layer "F.Cu") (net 5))
 (segment (start 130.851 40.249) (end 127.43253 40.249) (width 0.2) (layer "F.Cu") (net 5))
 (segment (start 129.7 49.02) (end 130.851 47.869) (width 0.2) (layer "F.Cu") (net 5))
 (segment (start 109 58.68153) (end 109 70.6) (width 0.2) (layer "F.Cu") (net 5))
 (via (at 109 70.6) (size 0.6) (drill 0.3) (layers "F.Cu" "B.Cu") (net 5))
 (segment (start 102.143274 95.691) (end 101.634 96.200274) (width 0.2) (layer "B.Cu") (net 5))
 (segment (start 101.634 96.200274) (end 101.634 98.673943) (width 0.2) (layer "B.Cu") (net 5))
 (segment (start 109 70.6) (end 109 92.7) (width 0.2) (layer "B.Cu") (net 5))
 (segment (start 109 92.7) (end 106.009 95.691) (width 0.2) (layer "B.Cu") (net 5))
 (segment (start 102.655057 99.695) (end 104.4 99.695) (width 0.2) (layer "B.Cu") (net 5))
 (segment (start 106.009 95.691) (end 102.143274 95.691) (width 0.2) (layer "B.Cu") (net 5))
 (segment (start 101.634 98.673943) (end 102.655057 99.695) (width 0.2) (layer "B.Cu") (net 5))
 (segment (start 129.7 43.94) (end 125.441 48.199) (width 0.2) (layer "F.Cu") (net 3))
 (segment (start 125.441 48.199) (end 125.441 57.300314) (width 0.2) (layer "F.Cu") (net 3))
 (segment (start 124.620314 64.129629) (end 117.774943 70.975) (width 0.2) (layer "F.Cu") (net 3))
 (segment (start 118.577 108.792) (end 119.64 109.855) (width 0.2) (layer "F.Cu") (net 3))
 (segment (start 104.37369 103.712) (end 117.07369 103.712) (width 0.2) (layer "F.Cu") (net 3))
 (segment (start 124.620314 58.121) (end 124.620314 64.129629) (width 0.2) (layer "F.Cu") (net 3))
 (segment (start 102.235 98.425) (end 102.235 101.57331) (width 0.2) (layer "F.Cu") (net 3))
 (segment (start 119.510527 106.053) (end 119.39869 106.053) (width 0.2) (layer "F.Cu") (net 3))
 (segment (start 118.577 106.87469) (end 118.577 108.792) (width 0.2) (layer "F.Cu") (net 3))
 (segment (start 102.235 101.57331) (end 104.37369 103.712) (width 0.2) (layer "F.Cu") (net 3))
 (segment (start 125.441 57.300314) (end 124.620314 58.121) (width 0.2) (layer "F.Cu") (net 3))
 (segment (start 117.774943 70.975) (end 110 70.975) (width 0.2) (layer "F.Cu") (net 3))
 (segment (start 117.07369 103.712) (end 119.41469 106.053) (width 0.2) (layer "F.Cu") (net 3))
 (segment (start 119.41469 106.053) (end 119.510527 106.053) (width 0.2) (layer "F.Cu") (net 3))
 (segment (start 119.39869 106.053) (end 118.577 106.87469) (width 0.2) (layer "F.Cu") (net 3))
 (via (at 102.235 98.425) (size 0.6) (drill 0.3) (layers "F.Cu" "B.Cu") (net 3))
 (via (at 110 70.975) (size 0.6) (drill 0.3) (layers "F.Cu" "B.Cu") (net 3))
 (segment (start 102.309374 96.092) (end 102.048 96.353374) (width 0.2) (layer "B.Cu") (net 3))
 (segment (start 110 70.975) (end 110 92.49121) (width 0.2) (layer "B.Cu") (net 3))
 (segment (start 102.048 96.353374) (end 102.048 98.238) (width 0.2) (layer "B.Cu") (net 3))
 (segment (start 106.39921 96.092) (end 102.309374 96.092) (width 0.2) (layer "B.Cu") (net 3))
 (segment (start 110 92.49121) (end 106.39921 96.092) (width 0.2) (layer "B.Cu") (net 3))
 (segment (start 102.048 98.238) (end 102.235 98.425) (width 0.2) (layer "B.Cu") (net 3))
 (segment (start 105.463 96.092) (end 105.463 93.437) (width 0.2) (layer "F.Cu") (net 4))
 (segment (start 105.463 93.437) (end 107.9 91) (width 0.2) (layer "F.Cu") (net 4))
 (segment (start 104.4 97.155) (end 105.463 96.092) (width 0.2) (layer "F.Cu") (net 4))
 (segment (start 107.9 91) (end 108.09511 90.80489) (width 0.2) (layer "F.Cu") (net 4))
 (segment (start 108.09511 90.80489) (end 111.40489 90.80489) (width 0.2) (layer "F.Cu") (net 4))
 (via (at 111.40489 90.80489) (size 0.6) (drill 0.3) (layers "F.Cu" "B.Cu") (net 4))
 (segment (start 128.488686 46.48) (end 129.7 46.48) (width 0.2) (layer "B.Cu") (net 4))
 (segment (start 111.40489 90.80489) (end 111.40489 63.563796) (width 0.2) (layer "B.Cu") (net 4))
 (segment (start 111.40489 63.563796) (end 128.488686 46.48) (width 0.2) (layer "B.Cu") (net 4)))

